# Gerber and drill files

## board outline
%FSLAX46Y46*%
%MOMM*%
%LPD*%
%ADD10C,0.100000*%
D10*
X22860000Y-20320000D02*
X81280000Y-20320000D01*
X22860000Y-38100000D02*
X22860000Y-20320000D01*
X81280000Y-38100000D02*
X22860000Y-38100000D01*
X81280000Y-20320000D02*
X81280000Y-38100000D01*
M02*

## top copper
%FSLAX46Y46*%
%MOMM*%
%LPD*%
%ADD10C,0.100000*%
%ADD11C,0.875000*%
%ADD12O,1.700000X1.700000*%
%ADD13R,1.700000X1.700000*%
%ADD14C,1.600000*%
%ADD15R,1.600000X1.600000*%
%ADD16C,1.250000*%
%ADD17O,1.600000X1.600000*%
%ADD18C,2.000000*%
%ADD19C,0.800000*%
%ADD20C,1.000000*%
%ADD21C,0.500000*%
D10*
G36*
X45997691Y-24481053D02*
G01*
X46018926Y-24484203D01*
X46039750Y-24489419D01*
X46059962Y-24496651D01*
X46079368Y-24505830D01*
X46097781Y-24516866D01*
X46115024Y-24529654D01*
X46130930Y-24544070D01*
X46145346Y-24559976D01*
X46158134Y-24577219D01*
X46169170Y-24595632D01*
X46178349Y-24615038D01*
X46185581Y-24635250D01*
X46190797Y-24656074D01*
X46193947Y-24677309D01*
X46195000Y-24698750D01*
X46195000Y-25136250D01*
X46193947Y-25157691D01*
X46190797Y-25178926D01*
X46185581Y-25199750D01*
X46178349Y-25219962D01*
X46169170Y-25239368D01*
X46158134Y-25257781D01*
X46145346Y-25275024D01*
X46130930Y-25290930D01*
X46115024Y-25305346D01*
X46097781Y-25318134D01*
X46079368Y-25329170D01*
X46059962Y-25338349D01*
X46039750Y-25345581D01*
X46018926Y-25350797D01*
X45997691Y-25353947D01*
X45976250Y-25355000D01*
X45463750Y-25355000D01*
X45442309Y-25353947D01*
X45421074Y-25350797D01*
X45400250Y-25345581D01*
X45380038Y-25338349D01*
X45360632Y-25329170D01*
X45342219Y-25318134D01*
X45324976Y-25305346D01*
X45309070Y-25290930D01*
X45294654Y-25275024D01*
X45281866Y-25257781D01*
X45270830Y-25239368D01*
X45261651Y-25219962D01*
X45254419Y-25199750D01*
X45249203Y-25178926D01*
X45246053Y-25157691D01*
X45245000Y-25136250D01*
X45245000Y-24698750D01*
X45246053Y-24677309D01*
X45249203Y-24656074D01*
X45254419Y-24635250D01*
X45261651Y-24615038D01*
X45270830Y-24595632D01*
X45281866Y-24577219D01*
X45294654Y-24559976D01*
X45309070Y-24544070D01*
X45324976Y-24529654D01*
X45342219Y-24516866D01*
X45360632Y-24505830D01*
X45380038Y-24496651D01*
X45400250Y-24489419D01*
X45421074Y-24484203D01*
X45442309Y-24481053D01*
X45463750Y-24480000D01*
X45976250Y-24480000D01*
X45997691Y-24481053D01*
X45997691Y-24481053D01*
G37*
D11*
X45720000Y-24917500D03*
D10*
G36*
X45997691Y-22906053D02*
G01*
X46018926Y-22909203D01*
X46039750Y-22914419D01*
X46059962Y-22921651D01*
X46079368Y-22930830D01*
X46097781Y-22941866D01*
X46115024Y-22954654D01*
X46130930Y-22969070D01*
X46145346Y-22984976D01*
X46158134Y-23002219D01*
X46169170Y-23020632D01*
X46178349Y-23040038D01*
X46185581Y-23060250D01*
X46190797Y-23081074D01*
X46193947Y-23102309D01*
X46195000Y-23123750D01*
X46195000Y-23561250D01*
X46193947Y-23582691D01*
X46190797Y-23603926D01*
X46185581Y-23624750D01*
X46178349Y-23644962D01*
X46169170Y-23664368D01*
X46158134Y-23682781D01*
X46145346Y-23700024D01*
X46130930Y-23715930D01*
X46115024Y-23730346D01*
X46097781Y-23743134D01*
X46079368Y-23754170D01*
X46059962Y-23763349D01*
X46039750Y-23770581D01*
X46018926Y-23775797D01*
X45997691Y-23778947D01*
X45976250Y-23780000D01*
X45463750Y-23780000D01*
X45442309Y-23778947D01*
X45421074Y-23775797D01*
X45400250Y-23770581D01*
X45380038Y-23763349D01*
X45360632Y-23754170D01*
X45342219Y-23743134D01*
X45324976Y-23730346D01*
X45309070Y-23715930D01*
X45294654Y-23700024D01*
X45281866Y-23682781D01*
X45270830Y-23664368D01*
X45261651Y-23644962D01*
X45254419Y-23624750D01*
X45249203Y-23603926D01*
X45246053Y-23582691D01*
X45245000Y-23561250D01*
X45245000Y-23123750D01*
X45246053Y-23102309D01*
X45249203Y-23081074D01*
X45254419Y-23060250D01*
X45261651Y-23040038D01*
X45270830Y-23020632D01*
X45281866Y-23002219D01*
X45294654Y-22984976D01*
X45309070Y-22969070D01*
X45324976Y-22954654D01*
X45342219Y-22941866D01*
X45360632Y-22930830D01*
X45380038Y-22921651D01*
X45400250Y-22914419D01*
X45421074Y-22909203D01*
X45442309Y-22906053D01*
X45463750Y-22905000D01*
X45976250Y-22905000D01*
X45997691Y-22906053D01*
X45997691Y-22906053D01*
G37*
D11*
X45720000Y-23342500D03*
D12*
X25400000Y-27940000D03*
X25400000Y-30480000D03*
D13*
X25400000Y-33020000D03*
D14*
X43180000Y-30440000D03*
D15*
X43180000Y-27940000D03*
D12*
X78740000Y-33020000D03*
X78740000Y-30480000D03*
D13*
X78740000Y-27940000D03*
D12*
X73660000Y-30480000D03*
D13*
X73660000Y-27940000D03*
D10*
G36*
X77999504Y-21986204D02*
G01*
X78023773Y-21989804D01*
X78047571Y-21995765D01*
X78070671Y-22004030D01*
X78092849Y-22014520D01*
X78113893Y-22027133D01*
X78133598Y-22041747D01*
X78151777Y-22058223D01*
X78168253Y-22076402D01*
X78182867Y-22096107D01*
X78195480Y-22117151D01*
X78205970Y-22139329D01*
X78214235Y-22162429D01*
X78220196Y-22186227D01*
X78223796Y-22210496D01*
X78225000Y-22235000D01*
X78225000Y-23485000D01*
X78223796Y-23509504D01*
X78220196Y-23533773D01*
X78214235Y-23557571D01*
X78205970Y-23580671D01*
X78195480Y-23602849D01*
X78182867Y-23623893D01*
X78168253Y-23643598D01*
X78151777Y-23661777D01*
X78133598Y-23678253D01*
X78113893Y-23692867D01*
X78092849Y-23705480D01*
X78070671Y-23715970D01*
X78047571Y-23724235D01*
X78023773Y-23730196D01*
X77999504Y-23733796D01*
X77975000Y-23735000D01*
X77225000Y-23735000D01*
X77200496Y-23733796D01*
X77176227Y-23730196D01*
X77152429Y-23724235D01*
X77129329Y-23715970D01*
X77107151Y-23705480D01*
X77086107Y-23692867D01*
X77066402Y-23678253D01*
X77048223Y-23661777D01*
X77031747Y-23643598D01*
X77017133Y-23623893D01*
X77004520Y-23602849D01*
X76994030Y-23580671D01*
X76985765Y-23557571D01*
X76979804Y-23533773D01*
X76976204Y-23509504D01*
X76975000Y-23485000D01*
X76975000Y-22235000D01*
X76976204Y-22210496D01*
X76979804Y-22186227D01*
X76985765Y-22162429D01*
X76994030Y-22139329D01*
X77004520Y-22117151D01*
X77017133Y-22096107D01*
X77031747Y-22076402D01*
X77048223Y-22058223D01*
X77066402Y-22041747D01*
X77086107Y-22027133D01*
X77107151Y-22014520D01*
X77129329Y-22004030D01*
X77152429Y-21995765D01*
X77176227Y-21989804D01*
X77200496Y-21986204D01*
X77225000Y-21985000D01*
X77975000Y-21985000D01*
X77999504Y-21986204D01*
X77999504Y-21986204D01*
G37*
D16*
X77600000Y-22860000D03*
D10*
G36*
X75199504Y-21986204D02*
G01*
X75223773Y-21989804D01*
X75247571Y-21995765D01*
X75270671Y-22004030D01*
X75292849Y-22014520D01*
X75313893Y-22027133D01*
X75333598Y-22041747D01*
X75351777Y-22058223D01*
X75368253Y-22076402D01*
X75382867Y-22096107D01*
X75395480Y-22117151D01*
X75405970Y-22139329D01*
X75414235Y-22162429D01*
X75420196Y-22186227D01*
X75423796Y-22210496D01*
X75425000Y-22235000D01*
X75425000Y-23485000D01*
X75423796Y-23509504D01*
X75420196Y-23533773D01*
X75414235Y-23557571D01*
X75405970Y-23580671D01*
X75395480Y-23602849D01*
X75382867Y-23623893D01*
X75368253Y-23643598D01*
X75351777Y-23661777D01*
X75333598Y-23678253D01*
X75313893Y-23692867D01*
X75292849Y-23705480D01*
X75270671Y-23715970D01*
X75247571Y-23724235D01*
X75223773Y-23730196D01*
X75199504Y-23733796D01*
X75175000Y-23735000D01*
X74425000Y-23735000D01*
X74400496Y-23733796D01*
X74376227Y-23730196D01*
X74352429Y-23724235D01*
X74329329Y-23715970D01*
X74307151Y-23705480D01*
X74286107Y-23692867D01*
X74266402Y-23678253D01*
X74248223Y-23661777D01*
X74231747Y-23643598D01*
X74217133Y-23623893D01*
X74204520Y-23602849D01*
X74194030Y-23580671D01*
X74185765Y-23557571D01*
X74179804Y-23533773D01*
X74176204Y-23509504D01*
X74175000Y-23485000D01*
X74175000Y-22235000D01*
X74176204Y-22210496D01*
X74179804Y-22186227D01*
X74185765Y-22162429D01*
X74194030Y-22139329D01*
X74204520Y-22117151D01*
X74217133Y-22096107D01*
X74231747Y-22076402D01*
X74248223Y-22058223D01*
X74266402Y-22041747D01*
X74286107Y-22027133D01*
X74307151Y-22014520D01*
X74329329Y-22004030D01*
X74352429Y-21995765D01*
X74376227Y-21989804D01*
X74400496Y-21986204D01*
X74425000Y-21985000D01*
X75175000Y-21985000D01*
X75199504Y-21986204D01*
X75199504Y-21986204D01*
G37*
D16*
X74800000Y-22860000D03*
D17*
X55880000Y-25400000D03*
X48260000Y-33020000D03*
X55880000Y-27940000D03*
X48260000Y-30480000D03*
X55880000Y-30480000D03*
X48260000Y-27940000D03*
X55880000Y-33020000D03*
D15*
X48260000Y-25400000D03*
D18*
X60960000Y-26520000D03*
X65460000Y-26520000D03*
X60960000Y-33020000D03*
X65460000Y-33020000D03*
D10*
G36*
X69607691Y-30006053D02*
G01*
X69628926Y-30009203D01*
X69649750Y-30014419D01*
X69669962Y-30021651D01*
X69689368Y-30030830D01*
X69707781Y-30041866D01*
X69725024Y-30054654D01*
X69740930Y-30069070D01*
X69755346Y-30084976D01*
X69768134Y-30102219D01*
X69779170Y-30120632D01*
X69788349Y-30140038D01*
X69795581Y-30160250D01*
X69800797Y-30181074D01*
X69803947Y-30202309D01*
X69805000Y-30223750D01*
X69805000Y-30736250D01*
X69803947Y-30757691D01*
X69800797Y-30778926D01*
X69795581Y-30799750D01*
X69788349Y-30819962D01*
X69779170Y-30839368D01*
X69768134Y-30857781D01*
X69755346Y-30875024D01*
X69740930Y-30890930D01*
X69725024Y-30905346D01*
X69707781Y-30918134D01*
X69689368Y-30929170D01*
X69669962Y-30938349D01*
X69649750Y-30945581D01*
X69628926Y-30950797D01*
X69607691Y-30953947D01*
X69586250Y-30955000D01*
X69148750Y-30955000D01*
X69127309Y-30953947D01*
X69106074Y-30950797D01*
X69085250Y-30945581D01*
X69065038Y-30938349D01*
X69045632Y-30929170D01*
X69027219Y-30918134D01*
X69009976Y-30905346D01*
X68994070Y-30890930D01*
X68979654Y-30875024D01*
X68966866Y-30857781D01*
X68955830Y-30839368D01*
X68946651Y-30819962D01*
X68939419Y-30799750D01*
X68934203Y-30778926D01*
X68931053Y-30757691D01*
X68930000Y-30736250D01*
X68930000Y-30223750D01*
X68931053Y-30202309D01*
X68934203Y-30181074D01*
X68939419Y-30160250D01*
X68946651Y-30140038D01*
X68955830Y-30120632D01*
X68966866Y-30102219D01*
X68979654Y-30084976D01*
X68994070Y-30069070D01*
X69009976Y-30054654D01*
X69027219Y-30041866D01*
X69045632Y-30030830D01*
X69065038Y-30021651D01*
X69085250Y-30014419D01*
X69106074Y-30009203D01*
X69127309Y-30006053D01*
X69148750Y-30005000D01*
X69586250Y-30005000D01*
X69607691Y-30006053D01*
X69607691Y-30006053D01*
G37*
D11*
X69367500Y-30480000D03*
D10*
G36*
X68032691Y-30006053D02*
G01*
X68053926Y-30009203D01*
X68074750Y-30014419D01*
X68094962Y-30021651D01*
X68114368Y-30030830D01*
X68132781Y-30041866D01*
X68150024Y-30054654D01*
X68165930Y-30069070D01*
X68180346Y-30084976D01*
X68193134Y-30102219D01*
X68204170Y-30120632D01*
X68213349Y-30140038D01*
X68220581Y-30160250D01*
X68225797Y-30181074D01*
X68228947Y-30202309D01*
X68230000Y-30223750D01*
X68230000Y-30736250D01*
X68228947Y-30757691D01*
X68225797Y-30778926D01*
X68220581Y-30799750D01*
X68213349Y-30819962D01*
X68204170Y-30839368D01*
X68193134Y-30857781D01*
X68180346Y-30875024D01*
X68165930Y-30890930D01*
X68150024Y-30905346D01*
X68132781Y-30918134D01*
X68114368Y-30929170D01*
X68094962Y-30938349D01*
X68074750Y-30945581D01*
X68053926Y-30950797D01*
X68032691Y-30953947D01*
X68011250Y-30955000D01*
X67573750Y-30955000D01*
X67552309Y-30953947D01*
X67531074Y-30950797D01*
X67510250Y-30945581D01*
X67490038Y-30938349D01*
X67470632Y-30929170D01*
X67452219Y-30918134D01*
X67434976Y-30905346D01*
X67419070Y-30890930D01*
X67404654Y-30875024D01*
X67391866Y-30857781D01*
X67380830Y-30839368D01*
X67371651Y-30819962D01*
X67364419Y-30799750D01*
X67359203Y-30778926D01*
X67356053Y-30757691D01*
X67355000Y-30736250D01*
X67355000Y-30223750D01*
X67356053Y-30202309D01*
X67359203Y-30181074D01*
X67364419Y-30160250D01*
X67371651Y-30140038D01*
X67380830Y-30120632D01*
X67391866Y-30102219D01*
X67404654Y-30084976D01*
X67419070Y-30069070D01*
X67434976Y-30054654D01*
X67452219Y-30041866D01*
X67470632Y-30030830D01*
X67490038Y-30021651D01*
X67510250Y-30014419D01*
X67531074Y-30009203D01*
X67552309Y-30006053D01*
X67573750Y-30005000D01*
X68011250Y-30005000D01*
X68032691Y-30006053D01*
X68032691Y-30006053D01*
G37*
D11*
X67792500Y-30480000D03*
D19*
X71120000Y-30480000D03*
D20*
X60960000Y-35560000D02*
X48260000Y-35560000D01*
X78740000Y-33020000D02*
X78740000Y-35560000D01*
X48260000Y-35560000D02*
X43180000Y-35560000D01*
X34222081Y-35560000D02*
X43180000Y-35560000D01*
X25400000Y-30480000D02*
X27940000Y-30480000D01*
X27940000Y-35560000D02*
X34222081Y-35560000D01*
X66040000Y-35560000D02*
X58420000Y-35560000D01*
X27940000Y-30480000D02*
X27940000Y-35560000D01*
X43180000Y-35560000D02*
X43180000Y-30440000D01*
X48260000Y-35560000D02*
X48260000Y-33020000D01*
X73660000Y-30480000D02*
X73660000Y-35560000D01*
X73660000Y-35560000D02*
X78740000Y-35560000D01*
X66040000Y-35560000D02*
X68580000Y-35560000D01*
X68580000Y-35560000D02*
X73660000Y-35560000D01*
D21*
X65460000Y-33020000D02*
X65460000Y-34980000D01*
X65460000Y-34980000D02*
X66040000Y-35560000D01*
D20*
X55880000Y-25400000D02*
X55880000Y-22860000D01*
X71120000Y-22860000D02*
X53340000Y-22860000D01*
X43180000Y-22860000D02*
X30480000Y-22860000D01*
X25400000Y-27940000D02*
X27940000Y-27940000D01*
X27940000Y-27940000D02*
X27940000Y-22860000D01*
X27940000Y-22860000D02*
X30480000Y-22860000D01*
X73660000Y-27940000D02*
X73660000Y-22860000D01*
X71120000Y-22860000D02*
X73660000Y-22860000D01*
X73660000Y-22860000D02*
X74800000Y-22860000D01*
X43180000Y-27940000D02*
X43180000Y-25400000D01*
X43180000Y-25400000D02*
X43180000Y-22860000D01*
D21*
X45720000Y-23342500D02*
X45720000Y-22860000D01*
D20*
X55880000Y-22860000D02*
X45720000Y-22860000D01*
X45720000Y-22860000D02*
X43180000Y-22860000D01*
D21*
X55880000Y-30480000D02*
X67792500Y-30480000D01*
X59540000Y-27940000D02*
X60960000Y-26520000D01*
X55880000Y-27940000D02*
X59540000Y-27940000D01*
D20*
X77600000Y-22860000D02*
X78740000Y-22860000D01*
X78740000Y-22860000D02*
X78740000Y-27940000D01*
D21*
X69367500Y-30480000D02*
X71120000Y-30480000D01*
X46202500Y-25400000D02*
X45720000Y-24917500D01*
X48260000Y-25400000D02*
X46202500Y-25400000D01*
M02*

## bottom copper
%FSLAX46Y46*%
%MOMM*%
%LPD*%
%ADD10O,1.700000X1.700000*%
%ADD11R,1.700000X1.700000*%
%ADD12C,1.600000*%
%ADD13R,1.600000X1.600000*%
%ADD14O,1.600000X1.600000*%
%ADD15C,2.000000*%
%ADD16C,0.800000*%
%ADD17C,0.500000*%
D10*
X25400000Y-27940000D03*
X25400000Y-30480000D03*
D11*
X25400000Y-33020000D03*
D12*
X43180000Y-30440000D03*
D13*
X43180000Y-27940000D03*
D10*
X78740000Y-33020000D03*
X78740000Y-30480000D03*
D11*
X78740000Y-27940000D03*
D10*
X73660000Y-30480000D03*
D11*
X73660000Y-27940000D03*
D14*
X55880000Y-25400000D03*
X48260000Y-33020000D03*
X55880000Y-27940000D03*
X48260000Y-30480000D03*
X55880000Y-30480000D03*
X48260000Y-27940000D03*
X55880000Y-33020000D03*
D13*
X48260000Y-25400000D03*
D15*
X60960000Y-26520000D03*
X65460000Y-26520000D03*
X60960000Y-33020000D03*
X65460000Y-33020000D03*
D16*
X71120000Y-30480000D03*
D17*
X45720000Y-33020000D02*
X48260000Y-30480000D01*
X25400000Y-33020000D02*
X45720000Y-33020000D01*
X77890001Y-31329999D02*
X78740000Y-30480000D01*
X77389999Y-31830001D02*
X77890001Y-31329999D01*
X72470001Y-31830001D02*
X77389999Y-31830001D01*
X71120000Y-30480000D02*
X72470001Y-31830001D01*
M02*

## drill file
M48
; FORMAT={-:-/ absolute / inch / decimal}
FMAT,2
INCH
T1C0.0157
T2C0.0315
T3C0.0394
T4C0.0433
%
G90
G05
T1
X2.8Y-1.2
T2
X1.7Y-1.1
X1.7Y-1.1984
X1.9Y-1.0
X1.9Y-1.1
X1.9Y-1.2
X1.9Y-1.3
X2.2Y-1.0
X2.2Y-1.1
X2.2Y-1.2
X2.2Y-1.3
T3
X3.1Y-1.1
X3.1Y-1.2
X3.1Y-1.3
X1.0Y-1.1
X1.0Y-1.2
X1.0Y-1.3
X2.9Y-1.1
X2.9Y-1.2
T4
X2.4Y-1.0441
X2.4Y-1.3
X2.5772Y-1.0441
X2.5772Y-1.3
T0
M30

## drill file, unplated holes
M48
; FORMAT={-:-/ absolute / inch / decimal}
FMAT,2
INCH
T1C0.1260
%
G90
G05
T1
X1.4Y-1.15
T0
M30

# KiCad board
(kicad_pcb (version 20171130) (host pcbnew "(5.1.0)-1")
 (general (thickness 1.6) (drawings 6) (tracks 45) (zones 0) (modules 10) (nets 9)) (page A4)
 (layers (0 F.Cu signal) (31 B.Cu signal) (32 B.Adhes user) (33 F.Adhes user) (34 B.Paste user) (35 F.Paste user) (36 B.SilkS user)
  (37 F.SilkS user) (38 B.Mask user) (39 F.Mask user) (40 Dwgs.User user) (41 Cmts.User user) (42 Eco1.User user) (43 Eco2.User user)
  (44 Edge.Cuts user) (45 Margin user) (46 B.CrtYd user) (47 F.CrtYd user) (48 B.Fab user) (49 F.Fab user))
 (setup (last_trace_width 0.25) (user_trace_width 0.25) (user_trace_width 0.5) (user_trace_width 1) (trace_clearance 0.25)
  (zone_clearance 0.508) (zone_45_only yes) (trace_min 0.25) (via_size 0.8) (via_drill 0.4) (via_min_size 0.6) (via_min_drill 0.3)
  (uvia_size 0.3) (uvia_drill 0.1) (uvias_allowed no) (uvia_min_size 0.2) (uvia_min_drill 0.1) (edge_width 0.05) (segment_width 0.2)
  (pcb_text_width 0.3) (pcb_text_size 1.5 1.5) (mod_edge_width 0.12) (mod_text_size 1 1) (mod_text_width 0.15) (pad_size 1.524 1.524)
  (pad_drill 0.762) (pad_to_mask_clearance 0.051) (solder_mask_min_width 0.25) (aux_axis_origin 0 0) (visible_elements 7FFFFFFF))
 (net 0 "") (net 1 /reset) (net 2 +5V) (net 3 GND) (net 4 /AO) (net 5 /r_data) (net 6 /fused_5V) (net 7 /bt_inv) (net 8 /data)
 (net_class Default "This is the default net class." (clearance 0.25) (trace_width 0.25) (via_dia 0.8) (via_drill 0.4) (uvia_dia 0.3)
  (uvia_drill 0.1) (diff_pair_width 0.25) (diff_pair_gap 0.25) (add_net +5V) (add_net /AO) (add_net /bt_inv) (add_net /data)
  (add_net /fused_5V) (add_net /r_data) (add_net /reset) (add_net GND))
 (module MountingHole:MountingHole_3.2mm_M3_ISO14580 (layer F.Cu) (at 35.56 29.21)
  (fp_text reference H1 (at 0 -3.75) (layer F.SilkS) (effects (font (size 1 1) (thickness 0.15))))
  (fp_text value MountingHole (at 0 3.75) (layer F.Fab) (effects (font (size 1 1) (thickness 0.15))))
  (pad 1 np_thru_hole circle (at 0 0) (size 3.2 3.2) (drill 3.2) (layers *.Cu *.Mask)))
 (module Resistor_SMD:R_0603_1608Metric (layer F.Cu) (at 45.72 24.13 270)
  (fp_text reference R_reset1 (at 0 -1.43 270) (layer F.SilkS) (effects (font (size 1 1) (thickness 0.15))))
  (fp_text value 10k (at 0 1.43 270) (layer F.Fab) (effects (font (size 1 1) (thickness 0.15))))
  (pad 2 smd roundrect (at 0.7875 0 270) (size 0.875 0.95) (layers F.Cu F.Paste F.Mask) (roundrect_rratio 0.25) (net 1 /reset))
  (pad 1 smd roundrect (at -0.7875 0 270) (size 0.875 0.95) (layers F.Cu F.Paste F.Mask) (roundrect_rratio 0.25) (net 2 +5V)))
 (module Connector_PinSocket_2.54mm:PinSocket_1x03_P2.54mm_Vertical (layer F.Cu) (at 25.4 33.02 180)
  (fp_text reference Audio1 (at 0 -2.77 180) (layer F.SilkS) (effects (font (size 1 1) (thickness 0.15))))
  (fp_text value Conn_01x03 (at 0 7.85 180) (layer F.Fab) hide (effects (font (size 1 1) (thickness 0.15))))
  (pad 3 thru_hole oval (at 0 5.08 180) (size 1.7 1.7) (drill 1) (layers *.Cu *.Mask) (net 2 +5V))
  (pad 2 thru_hole oval (at 0 2.54 180) (size 1.7 1.7) (drill 1) (layers *.Cu *.Mask) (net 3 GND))
  (pad 1 thru_hole rect (at 0 0 180) (size 1.7 1.7) (drill 1) (layers *.Cu *.Mask) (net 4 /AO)))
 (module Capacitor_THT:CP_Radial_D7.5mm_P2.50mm (layer F.Cu) (at 43.18 27.94 270)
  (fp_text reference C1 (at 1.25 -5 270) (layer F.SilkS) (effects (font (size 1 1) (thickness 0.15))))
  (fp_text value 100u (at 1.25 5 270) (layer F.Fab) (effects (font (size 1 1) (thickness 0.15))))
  (pad 2 thru_hole circle (at 2.5 0 270) (size 1.6 1.6) (drill 0.8) (layers *.Cu *.Mask) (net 3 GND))
  (pad 1 thru_hole rect (at 0 0 270) (size 1.6 1.6) (drill 0.8) (layers *.Cu *.Mask) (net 2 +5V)))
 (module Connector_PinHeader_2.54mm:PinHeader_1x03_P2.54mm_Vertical (layer B.Cu) (at 78.74 27.94 180)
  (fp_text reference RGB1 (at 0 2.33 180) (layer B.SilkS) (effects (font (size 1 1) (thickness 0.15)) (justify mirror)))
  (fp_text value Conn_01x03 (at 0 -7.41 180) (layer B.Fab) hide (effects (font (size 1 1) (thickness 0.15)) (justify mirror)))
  (pad 3 thru_hole oval (at 0 -5.08 180) (size 1.7 1.7) (drill 1) (layers *.Cu *.Mask) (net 3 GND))
  (pad 2 thru_hole oval (at 0 -2.54 180) (size 1.7 1.7) (drill 1) (layers *.Cu *.Mask) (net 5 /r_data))
  (pad 1 thru_hole rect (at 0 0 180) (size 1.7 1.7) (drill 1) (layers *.Cu *.Mask) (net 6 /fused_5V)))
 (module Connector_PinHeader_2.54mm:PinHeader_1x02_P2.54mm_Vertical (layer F.Cu) (at 73.66 27.94)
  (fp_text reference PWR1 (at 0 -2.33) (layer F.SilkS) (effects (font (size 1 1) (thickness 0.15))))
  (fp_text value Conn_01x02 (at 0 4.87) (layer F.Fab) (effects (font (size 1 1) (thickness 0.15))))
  (pad 2 thru_hole oval (at 0 2.54) (size 1.7 1.7) (drill 1) (layers *.Cu *.Mask) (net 3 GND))
  (pad 1 thru_hole rect (at 0 0) (size 1.7 1.7) (drill 1) (layers *.Cu *.Mask) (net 2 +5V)))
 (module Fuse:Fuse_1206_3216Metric (layer F.Cu) (at 76.2 22.86)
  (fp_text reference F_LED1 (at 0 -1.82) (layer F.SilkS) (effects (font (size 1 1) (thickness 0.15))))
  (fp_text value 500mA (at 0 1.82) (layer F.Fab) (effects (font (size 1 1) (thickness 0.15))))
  (pad 2 smd roundrect (at 1.4 0) (size 1.25 1.75) (layers F.Cu F.Paste F.Mask) (roundrect_rratio 0.2) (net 6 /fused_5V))
  (pad 1 smd roundrect (at -1.4 0) (size 1.25 1.75) (layers F.Cu F.Paste F.Mask) (roundrect_rratio 0.2) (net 2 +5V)))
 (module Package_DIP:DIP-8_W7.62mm (layer F.Cu) (at 48.26 25.4)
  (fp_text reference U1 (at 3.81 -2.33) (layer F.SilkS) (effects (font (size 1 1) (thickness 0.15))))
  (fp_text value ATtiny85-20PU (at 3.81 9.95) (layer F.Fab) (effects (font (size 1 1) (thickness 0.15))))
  (pad 8 thru_hole oval (at 7.62 0) (size 1.6 1.6) (drill 0.8) (layers *.Cu *.Mask) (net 2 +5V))
  (pad 4 thru_hole oval (at 0 7.62) (size 1.6 1.6) (drill 0.8) (layers *.Cu *.Mask) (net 3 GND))
  (pad 7 thru_hole oval (at 7.62 2.54) (size 1.6 1.6) (drill 0.8) (layers *.Cu *.Mask) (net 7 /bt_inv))
  (pad 3 thru_hole oval (at 0 5.08) (size 1.6 1.6) (drill 0.8) (layers *.Cu *.Mask) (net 4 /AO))
  (pad 6 thru_hole oval (at 7.62 5.08) (size 1.6 1.6) (drill 0.8) (layers *.Cu *.Mask) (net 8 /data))
  (pad 2 thru_hole oval (at 0 2.54) (size 1.6 1.6) (drill 0.8) (layers *.Cu *.Mask))
  (pad 5 thru_hole oval (at 7.62 7.62) (size 1.6 1.6) (drill 0.8) (layers *.Cu *.Mask))
  (pad 1 thru_hole rect (at 0 0) (size 1.6 1.6) (drill 0.8) (layers *.Cu *.Mask) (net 1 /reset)))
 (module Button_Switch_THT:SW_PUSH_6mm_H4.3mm (layer F.Cu) (at 60.96 33.02 90)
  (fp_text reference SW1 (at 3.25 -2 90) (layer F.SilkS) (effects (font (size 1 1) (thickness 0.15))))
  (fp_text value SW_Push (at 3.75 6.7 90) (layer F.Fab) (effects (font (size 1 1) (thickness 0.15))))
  (pad 1 thru_hole circle (at 6.5 0 180) (size 2 2) (drill 1.1) (layers *.Cu *.Mask) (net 7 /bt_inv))
  (pad 2 thru_hole circle (at 6.5 4.5 180) (size 2 2) (drill 1.1) (layers *.Cu *.Mask) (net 3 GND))
  (pad 1 thru_hole circle (at 0 0 180) (size 2 2) (drill 1.1) (layers *.Cu *.Mask) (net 7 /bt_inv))
  (pad 2 thru_hole circle (at 0 4.5 180) (size 2 2) (drill 1.1) (layers *.Cu *.Mask) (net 3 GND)))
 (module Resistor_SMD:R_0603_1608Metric (layer F.Cu) (at 68.58 30.48)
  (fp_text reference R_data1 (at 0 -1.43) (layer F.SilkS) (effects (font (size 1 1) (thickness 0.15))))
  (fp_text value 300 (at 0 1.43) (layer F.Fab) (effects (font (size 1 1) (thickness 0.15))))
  (pad 2 smd roundrect (at 0.7875 0) (size 0.875 0.95) (layers F.Cu F.Paste F.Mask) (roundrect_rratio 0.25) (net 5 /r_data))
  (pad 1 smd roundrect (at -0.7875 0) (size 0.875 0.95) (layers F.Cu F.Paste F.Mask) (roundrect_rratio 0.25) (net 8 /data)))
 (gr_line (start 22.86 20.32) (end 81.28 20.32) (layer Edge.Cuts) (width 0.1))
 (gr_line (start 22.86 38.1) (end 22.86 20.32) (layer Edge.Cuts) (width 0.1))
 (gr_line (start 81.28 38.1) (end 22.86 38.1) (layer Edge.Cuts) (width 0.1))
 (gr_line (start 81.28 20.32) (end 81.28 38.1) (layer Edge.Cuts) (width 0.1))
 (segment (start 60.96 35.56) (end 48.26 35.56) (width 1) (layer F.Cu) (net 3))
 (segment (start 78.74 33.02) (end 78.74 35.56) (width 1) (layer F.Cu) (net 3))
 (segment (start 48.26 35.56) (end 43.18 35.56) (width 1) (layer F.Cu) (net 3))
 (segment (start 34.222081 35.56) (end 43.18 35.56) (width 1) (layer F.Cu) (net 3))
 (segment (start 25.4 30.48) (end 27.94 30.48) (width 1) (layer F.Cu) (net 3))
 (segment (start 27.94 35.56) (end 34.222081 35.56) (width 1) (layer F.Cu) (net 3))
 (segment (start 66.04 35.56) (end 58.42 35.56) (width 1) (layer F.Cu) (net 3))
 (segment (start 27.94 30.48) (end 27.94 35.56) (width 1) (layer F.Cu) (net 3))
 (segment (start 43.18 35.56) (end 43.18 30.44) (width 1) (layer F.Cu) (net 3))
 (segment (start 48.26 35.56) (end 48.26 33.02) (width 1) (layer F.Cu) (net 3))
 (segment (start 73.66 30.48) (end 73.66 35.56) (width 1) (layer F.Cu) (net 3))
 (segment (start 73.66 35.56) (end 78.74 35.56) (width 1) (layer F.Cu) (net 3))
 (segment (start 66.04 35.56) (end 68.58 35.56) (width 1) (layer F.Cu) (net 3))
 (segment (start 68.58 35.56) (end 73.66 35.56) (width 1) (layer F.Cu) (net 3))
 (segment (start 65.46 33.02) (end 65.46 34.98) (width 0.5) (layer F.Cu) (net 3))
 (segment (start 65.46 34.98) (end 66.04 35.56) (width 0.5) (layer F.Cu) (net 3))
 (segment (start 55.88 25.4) (end 55.88 22.86) (width 1) (layer F.Cu) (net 2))
 (segment (start 71.12 22.86) (end 53.34 22.86) (width 1) (layer F.Cu) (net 2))
 (segment (start 43.18 22.86) (end 30.48 22.86) (width 1) (layer F.Cu) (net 2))
 (segment (start 25.4 27.94) (end 27.94 27.94) (width 1) (layer F.Cu) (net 2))
 (segment (start 27.94 27.94) (end 27.94 22.86) (width 1) (layer F.Cu) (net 2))
 (segment (start 27.94 22.86) (end 30.48 22.86) (width 1) (layer F.Cu) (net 2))
 (segment (start 73.66 27.94) (end 73.66 22.86) (width 1) (layer F.Cu) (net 2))
 (segment (start 71.12 22.86) (end 73.66 22.86) (width 1) (layer F.Cu) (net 2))
 (segment (start 73.66 22.86) (end 74.8 22.86) (width 1) (layer F.Cu) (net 2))
 (segment (start 43.18 27.94) (end 43.18 25.4) (width 1) (layer F.Cu) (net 2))
 (segment (start 43.18 25.4) (end 43.18 22.86) (width 1) (layer F.Cu) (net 2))
 (segment (start 45.72 23.3425) (end 45.72 22.86) (width 0.5) (layer F.Cu) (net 2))
 (segment (start 55.88 22.86) (end 45.72 22.86) (width 1) (layer F.Cu) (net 2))
 (segment (start 45.72 22.86) (end 43.18 22.86) (width 1) (layer F.Cu) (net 2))
 (segment (start 55.88 30.48) (end 67.7925 30.48) (width 0.5) (layer F.Cu) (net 8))
 (segment (start 59.54 27.94) (end 60.96 26.52) (width 0.5) (layer F.Cu) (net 7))
 (segment (start 55.88 27.94) (end 59.54 27.94) (width 0.5) (layer F.Cu) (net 7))
 (segment (start 45.72 33.02) (end 48.26 30.48) (width 0.5) (layer B.Cu) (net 4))
 (segment (start 25.4 33.02) (end 45.72 33.02) (width 0.5) (layer B.Cu) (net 4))
 (segment (start 77.6 22.86) (end 78.74 22.86) (width 1) (layer F.Cu) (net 6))
 (segment (start 78.74 22.86) (end 78.74 27.94) (width 1) (layer F.Cu) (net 6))
 (via (at 71.12 30.48) (size 0.8) (drill 0.4) (layers F.Cu B.Cu) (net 5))
 (segment (start 69.3675 30.48) (end 71.12 30.48) (width 0.5) (layer F.Cu) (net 5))
 (segment (start 77.890001 31.329999) (end 78.74 30.48) (width 0.5) (layer B.Cu) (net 5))
 (segment (start 77.389999 31.830001) (end 77.890001 31.329999) (width 0.5) (layer B.Cu) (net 5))
 (segment (start 72.470001 31.830001) (end 77.389999 31.830001) (width 0.5) (layer B.Cu) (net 5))
 (segment (start 71.12 30.48) (end 72.470001 31.830001) (width 0.5) (layer B.Cu) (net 5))
 (segment (start 46.2025 25.4) (end 45.72 24.9175) (width 0.5) (layer F.Cu) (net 1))
 (segment (start 48.26 25.4) (end 46.2025 25.4) (width 0.5) (layer F.Cu) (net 1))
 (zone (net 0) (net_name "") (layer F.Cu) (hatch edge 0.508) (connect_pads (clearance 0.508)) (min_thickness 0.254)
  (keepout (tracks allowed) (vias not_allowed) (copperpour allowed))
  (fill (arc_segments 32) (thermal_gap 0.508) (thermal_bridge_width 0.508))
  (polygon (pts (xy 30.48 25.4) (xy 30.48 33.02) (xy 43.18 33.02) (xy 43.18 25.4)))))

